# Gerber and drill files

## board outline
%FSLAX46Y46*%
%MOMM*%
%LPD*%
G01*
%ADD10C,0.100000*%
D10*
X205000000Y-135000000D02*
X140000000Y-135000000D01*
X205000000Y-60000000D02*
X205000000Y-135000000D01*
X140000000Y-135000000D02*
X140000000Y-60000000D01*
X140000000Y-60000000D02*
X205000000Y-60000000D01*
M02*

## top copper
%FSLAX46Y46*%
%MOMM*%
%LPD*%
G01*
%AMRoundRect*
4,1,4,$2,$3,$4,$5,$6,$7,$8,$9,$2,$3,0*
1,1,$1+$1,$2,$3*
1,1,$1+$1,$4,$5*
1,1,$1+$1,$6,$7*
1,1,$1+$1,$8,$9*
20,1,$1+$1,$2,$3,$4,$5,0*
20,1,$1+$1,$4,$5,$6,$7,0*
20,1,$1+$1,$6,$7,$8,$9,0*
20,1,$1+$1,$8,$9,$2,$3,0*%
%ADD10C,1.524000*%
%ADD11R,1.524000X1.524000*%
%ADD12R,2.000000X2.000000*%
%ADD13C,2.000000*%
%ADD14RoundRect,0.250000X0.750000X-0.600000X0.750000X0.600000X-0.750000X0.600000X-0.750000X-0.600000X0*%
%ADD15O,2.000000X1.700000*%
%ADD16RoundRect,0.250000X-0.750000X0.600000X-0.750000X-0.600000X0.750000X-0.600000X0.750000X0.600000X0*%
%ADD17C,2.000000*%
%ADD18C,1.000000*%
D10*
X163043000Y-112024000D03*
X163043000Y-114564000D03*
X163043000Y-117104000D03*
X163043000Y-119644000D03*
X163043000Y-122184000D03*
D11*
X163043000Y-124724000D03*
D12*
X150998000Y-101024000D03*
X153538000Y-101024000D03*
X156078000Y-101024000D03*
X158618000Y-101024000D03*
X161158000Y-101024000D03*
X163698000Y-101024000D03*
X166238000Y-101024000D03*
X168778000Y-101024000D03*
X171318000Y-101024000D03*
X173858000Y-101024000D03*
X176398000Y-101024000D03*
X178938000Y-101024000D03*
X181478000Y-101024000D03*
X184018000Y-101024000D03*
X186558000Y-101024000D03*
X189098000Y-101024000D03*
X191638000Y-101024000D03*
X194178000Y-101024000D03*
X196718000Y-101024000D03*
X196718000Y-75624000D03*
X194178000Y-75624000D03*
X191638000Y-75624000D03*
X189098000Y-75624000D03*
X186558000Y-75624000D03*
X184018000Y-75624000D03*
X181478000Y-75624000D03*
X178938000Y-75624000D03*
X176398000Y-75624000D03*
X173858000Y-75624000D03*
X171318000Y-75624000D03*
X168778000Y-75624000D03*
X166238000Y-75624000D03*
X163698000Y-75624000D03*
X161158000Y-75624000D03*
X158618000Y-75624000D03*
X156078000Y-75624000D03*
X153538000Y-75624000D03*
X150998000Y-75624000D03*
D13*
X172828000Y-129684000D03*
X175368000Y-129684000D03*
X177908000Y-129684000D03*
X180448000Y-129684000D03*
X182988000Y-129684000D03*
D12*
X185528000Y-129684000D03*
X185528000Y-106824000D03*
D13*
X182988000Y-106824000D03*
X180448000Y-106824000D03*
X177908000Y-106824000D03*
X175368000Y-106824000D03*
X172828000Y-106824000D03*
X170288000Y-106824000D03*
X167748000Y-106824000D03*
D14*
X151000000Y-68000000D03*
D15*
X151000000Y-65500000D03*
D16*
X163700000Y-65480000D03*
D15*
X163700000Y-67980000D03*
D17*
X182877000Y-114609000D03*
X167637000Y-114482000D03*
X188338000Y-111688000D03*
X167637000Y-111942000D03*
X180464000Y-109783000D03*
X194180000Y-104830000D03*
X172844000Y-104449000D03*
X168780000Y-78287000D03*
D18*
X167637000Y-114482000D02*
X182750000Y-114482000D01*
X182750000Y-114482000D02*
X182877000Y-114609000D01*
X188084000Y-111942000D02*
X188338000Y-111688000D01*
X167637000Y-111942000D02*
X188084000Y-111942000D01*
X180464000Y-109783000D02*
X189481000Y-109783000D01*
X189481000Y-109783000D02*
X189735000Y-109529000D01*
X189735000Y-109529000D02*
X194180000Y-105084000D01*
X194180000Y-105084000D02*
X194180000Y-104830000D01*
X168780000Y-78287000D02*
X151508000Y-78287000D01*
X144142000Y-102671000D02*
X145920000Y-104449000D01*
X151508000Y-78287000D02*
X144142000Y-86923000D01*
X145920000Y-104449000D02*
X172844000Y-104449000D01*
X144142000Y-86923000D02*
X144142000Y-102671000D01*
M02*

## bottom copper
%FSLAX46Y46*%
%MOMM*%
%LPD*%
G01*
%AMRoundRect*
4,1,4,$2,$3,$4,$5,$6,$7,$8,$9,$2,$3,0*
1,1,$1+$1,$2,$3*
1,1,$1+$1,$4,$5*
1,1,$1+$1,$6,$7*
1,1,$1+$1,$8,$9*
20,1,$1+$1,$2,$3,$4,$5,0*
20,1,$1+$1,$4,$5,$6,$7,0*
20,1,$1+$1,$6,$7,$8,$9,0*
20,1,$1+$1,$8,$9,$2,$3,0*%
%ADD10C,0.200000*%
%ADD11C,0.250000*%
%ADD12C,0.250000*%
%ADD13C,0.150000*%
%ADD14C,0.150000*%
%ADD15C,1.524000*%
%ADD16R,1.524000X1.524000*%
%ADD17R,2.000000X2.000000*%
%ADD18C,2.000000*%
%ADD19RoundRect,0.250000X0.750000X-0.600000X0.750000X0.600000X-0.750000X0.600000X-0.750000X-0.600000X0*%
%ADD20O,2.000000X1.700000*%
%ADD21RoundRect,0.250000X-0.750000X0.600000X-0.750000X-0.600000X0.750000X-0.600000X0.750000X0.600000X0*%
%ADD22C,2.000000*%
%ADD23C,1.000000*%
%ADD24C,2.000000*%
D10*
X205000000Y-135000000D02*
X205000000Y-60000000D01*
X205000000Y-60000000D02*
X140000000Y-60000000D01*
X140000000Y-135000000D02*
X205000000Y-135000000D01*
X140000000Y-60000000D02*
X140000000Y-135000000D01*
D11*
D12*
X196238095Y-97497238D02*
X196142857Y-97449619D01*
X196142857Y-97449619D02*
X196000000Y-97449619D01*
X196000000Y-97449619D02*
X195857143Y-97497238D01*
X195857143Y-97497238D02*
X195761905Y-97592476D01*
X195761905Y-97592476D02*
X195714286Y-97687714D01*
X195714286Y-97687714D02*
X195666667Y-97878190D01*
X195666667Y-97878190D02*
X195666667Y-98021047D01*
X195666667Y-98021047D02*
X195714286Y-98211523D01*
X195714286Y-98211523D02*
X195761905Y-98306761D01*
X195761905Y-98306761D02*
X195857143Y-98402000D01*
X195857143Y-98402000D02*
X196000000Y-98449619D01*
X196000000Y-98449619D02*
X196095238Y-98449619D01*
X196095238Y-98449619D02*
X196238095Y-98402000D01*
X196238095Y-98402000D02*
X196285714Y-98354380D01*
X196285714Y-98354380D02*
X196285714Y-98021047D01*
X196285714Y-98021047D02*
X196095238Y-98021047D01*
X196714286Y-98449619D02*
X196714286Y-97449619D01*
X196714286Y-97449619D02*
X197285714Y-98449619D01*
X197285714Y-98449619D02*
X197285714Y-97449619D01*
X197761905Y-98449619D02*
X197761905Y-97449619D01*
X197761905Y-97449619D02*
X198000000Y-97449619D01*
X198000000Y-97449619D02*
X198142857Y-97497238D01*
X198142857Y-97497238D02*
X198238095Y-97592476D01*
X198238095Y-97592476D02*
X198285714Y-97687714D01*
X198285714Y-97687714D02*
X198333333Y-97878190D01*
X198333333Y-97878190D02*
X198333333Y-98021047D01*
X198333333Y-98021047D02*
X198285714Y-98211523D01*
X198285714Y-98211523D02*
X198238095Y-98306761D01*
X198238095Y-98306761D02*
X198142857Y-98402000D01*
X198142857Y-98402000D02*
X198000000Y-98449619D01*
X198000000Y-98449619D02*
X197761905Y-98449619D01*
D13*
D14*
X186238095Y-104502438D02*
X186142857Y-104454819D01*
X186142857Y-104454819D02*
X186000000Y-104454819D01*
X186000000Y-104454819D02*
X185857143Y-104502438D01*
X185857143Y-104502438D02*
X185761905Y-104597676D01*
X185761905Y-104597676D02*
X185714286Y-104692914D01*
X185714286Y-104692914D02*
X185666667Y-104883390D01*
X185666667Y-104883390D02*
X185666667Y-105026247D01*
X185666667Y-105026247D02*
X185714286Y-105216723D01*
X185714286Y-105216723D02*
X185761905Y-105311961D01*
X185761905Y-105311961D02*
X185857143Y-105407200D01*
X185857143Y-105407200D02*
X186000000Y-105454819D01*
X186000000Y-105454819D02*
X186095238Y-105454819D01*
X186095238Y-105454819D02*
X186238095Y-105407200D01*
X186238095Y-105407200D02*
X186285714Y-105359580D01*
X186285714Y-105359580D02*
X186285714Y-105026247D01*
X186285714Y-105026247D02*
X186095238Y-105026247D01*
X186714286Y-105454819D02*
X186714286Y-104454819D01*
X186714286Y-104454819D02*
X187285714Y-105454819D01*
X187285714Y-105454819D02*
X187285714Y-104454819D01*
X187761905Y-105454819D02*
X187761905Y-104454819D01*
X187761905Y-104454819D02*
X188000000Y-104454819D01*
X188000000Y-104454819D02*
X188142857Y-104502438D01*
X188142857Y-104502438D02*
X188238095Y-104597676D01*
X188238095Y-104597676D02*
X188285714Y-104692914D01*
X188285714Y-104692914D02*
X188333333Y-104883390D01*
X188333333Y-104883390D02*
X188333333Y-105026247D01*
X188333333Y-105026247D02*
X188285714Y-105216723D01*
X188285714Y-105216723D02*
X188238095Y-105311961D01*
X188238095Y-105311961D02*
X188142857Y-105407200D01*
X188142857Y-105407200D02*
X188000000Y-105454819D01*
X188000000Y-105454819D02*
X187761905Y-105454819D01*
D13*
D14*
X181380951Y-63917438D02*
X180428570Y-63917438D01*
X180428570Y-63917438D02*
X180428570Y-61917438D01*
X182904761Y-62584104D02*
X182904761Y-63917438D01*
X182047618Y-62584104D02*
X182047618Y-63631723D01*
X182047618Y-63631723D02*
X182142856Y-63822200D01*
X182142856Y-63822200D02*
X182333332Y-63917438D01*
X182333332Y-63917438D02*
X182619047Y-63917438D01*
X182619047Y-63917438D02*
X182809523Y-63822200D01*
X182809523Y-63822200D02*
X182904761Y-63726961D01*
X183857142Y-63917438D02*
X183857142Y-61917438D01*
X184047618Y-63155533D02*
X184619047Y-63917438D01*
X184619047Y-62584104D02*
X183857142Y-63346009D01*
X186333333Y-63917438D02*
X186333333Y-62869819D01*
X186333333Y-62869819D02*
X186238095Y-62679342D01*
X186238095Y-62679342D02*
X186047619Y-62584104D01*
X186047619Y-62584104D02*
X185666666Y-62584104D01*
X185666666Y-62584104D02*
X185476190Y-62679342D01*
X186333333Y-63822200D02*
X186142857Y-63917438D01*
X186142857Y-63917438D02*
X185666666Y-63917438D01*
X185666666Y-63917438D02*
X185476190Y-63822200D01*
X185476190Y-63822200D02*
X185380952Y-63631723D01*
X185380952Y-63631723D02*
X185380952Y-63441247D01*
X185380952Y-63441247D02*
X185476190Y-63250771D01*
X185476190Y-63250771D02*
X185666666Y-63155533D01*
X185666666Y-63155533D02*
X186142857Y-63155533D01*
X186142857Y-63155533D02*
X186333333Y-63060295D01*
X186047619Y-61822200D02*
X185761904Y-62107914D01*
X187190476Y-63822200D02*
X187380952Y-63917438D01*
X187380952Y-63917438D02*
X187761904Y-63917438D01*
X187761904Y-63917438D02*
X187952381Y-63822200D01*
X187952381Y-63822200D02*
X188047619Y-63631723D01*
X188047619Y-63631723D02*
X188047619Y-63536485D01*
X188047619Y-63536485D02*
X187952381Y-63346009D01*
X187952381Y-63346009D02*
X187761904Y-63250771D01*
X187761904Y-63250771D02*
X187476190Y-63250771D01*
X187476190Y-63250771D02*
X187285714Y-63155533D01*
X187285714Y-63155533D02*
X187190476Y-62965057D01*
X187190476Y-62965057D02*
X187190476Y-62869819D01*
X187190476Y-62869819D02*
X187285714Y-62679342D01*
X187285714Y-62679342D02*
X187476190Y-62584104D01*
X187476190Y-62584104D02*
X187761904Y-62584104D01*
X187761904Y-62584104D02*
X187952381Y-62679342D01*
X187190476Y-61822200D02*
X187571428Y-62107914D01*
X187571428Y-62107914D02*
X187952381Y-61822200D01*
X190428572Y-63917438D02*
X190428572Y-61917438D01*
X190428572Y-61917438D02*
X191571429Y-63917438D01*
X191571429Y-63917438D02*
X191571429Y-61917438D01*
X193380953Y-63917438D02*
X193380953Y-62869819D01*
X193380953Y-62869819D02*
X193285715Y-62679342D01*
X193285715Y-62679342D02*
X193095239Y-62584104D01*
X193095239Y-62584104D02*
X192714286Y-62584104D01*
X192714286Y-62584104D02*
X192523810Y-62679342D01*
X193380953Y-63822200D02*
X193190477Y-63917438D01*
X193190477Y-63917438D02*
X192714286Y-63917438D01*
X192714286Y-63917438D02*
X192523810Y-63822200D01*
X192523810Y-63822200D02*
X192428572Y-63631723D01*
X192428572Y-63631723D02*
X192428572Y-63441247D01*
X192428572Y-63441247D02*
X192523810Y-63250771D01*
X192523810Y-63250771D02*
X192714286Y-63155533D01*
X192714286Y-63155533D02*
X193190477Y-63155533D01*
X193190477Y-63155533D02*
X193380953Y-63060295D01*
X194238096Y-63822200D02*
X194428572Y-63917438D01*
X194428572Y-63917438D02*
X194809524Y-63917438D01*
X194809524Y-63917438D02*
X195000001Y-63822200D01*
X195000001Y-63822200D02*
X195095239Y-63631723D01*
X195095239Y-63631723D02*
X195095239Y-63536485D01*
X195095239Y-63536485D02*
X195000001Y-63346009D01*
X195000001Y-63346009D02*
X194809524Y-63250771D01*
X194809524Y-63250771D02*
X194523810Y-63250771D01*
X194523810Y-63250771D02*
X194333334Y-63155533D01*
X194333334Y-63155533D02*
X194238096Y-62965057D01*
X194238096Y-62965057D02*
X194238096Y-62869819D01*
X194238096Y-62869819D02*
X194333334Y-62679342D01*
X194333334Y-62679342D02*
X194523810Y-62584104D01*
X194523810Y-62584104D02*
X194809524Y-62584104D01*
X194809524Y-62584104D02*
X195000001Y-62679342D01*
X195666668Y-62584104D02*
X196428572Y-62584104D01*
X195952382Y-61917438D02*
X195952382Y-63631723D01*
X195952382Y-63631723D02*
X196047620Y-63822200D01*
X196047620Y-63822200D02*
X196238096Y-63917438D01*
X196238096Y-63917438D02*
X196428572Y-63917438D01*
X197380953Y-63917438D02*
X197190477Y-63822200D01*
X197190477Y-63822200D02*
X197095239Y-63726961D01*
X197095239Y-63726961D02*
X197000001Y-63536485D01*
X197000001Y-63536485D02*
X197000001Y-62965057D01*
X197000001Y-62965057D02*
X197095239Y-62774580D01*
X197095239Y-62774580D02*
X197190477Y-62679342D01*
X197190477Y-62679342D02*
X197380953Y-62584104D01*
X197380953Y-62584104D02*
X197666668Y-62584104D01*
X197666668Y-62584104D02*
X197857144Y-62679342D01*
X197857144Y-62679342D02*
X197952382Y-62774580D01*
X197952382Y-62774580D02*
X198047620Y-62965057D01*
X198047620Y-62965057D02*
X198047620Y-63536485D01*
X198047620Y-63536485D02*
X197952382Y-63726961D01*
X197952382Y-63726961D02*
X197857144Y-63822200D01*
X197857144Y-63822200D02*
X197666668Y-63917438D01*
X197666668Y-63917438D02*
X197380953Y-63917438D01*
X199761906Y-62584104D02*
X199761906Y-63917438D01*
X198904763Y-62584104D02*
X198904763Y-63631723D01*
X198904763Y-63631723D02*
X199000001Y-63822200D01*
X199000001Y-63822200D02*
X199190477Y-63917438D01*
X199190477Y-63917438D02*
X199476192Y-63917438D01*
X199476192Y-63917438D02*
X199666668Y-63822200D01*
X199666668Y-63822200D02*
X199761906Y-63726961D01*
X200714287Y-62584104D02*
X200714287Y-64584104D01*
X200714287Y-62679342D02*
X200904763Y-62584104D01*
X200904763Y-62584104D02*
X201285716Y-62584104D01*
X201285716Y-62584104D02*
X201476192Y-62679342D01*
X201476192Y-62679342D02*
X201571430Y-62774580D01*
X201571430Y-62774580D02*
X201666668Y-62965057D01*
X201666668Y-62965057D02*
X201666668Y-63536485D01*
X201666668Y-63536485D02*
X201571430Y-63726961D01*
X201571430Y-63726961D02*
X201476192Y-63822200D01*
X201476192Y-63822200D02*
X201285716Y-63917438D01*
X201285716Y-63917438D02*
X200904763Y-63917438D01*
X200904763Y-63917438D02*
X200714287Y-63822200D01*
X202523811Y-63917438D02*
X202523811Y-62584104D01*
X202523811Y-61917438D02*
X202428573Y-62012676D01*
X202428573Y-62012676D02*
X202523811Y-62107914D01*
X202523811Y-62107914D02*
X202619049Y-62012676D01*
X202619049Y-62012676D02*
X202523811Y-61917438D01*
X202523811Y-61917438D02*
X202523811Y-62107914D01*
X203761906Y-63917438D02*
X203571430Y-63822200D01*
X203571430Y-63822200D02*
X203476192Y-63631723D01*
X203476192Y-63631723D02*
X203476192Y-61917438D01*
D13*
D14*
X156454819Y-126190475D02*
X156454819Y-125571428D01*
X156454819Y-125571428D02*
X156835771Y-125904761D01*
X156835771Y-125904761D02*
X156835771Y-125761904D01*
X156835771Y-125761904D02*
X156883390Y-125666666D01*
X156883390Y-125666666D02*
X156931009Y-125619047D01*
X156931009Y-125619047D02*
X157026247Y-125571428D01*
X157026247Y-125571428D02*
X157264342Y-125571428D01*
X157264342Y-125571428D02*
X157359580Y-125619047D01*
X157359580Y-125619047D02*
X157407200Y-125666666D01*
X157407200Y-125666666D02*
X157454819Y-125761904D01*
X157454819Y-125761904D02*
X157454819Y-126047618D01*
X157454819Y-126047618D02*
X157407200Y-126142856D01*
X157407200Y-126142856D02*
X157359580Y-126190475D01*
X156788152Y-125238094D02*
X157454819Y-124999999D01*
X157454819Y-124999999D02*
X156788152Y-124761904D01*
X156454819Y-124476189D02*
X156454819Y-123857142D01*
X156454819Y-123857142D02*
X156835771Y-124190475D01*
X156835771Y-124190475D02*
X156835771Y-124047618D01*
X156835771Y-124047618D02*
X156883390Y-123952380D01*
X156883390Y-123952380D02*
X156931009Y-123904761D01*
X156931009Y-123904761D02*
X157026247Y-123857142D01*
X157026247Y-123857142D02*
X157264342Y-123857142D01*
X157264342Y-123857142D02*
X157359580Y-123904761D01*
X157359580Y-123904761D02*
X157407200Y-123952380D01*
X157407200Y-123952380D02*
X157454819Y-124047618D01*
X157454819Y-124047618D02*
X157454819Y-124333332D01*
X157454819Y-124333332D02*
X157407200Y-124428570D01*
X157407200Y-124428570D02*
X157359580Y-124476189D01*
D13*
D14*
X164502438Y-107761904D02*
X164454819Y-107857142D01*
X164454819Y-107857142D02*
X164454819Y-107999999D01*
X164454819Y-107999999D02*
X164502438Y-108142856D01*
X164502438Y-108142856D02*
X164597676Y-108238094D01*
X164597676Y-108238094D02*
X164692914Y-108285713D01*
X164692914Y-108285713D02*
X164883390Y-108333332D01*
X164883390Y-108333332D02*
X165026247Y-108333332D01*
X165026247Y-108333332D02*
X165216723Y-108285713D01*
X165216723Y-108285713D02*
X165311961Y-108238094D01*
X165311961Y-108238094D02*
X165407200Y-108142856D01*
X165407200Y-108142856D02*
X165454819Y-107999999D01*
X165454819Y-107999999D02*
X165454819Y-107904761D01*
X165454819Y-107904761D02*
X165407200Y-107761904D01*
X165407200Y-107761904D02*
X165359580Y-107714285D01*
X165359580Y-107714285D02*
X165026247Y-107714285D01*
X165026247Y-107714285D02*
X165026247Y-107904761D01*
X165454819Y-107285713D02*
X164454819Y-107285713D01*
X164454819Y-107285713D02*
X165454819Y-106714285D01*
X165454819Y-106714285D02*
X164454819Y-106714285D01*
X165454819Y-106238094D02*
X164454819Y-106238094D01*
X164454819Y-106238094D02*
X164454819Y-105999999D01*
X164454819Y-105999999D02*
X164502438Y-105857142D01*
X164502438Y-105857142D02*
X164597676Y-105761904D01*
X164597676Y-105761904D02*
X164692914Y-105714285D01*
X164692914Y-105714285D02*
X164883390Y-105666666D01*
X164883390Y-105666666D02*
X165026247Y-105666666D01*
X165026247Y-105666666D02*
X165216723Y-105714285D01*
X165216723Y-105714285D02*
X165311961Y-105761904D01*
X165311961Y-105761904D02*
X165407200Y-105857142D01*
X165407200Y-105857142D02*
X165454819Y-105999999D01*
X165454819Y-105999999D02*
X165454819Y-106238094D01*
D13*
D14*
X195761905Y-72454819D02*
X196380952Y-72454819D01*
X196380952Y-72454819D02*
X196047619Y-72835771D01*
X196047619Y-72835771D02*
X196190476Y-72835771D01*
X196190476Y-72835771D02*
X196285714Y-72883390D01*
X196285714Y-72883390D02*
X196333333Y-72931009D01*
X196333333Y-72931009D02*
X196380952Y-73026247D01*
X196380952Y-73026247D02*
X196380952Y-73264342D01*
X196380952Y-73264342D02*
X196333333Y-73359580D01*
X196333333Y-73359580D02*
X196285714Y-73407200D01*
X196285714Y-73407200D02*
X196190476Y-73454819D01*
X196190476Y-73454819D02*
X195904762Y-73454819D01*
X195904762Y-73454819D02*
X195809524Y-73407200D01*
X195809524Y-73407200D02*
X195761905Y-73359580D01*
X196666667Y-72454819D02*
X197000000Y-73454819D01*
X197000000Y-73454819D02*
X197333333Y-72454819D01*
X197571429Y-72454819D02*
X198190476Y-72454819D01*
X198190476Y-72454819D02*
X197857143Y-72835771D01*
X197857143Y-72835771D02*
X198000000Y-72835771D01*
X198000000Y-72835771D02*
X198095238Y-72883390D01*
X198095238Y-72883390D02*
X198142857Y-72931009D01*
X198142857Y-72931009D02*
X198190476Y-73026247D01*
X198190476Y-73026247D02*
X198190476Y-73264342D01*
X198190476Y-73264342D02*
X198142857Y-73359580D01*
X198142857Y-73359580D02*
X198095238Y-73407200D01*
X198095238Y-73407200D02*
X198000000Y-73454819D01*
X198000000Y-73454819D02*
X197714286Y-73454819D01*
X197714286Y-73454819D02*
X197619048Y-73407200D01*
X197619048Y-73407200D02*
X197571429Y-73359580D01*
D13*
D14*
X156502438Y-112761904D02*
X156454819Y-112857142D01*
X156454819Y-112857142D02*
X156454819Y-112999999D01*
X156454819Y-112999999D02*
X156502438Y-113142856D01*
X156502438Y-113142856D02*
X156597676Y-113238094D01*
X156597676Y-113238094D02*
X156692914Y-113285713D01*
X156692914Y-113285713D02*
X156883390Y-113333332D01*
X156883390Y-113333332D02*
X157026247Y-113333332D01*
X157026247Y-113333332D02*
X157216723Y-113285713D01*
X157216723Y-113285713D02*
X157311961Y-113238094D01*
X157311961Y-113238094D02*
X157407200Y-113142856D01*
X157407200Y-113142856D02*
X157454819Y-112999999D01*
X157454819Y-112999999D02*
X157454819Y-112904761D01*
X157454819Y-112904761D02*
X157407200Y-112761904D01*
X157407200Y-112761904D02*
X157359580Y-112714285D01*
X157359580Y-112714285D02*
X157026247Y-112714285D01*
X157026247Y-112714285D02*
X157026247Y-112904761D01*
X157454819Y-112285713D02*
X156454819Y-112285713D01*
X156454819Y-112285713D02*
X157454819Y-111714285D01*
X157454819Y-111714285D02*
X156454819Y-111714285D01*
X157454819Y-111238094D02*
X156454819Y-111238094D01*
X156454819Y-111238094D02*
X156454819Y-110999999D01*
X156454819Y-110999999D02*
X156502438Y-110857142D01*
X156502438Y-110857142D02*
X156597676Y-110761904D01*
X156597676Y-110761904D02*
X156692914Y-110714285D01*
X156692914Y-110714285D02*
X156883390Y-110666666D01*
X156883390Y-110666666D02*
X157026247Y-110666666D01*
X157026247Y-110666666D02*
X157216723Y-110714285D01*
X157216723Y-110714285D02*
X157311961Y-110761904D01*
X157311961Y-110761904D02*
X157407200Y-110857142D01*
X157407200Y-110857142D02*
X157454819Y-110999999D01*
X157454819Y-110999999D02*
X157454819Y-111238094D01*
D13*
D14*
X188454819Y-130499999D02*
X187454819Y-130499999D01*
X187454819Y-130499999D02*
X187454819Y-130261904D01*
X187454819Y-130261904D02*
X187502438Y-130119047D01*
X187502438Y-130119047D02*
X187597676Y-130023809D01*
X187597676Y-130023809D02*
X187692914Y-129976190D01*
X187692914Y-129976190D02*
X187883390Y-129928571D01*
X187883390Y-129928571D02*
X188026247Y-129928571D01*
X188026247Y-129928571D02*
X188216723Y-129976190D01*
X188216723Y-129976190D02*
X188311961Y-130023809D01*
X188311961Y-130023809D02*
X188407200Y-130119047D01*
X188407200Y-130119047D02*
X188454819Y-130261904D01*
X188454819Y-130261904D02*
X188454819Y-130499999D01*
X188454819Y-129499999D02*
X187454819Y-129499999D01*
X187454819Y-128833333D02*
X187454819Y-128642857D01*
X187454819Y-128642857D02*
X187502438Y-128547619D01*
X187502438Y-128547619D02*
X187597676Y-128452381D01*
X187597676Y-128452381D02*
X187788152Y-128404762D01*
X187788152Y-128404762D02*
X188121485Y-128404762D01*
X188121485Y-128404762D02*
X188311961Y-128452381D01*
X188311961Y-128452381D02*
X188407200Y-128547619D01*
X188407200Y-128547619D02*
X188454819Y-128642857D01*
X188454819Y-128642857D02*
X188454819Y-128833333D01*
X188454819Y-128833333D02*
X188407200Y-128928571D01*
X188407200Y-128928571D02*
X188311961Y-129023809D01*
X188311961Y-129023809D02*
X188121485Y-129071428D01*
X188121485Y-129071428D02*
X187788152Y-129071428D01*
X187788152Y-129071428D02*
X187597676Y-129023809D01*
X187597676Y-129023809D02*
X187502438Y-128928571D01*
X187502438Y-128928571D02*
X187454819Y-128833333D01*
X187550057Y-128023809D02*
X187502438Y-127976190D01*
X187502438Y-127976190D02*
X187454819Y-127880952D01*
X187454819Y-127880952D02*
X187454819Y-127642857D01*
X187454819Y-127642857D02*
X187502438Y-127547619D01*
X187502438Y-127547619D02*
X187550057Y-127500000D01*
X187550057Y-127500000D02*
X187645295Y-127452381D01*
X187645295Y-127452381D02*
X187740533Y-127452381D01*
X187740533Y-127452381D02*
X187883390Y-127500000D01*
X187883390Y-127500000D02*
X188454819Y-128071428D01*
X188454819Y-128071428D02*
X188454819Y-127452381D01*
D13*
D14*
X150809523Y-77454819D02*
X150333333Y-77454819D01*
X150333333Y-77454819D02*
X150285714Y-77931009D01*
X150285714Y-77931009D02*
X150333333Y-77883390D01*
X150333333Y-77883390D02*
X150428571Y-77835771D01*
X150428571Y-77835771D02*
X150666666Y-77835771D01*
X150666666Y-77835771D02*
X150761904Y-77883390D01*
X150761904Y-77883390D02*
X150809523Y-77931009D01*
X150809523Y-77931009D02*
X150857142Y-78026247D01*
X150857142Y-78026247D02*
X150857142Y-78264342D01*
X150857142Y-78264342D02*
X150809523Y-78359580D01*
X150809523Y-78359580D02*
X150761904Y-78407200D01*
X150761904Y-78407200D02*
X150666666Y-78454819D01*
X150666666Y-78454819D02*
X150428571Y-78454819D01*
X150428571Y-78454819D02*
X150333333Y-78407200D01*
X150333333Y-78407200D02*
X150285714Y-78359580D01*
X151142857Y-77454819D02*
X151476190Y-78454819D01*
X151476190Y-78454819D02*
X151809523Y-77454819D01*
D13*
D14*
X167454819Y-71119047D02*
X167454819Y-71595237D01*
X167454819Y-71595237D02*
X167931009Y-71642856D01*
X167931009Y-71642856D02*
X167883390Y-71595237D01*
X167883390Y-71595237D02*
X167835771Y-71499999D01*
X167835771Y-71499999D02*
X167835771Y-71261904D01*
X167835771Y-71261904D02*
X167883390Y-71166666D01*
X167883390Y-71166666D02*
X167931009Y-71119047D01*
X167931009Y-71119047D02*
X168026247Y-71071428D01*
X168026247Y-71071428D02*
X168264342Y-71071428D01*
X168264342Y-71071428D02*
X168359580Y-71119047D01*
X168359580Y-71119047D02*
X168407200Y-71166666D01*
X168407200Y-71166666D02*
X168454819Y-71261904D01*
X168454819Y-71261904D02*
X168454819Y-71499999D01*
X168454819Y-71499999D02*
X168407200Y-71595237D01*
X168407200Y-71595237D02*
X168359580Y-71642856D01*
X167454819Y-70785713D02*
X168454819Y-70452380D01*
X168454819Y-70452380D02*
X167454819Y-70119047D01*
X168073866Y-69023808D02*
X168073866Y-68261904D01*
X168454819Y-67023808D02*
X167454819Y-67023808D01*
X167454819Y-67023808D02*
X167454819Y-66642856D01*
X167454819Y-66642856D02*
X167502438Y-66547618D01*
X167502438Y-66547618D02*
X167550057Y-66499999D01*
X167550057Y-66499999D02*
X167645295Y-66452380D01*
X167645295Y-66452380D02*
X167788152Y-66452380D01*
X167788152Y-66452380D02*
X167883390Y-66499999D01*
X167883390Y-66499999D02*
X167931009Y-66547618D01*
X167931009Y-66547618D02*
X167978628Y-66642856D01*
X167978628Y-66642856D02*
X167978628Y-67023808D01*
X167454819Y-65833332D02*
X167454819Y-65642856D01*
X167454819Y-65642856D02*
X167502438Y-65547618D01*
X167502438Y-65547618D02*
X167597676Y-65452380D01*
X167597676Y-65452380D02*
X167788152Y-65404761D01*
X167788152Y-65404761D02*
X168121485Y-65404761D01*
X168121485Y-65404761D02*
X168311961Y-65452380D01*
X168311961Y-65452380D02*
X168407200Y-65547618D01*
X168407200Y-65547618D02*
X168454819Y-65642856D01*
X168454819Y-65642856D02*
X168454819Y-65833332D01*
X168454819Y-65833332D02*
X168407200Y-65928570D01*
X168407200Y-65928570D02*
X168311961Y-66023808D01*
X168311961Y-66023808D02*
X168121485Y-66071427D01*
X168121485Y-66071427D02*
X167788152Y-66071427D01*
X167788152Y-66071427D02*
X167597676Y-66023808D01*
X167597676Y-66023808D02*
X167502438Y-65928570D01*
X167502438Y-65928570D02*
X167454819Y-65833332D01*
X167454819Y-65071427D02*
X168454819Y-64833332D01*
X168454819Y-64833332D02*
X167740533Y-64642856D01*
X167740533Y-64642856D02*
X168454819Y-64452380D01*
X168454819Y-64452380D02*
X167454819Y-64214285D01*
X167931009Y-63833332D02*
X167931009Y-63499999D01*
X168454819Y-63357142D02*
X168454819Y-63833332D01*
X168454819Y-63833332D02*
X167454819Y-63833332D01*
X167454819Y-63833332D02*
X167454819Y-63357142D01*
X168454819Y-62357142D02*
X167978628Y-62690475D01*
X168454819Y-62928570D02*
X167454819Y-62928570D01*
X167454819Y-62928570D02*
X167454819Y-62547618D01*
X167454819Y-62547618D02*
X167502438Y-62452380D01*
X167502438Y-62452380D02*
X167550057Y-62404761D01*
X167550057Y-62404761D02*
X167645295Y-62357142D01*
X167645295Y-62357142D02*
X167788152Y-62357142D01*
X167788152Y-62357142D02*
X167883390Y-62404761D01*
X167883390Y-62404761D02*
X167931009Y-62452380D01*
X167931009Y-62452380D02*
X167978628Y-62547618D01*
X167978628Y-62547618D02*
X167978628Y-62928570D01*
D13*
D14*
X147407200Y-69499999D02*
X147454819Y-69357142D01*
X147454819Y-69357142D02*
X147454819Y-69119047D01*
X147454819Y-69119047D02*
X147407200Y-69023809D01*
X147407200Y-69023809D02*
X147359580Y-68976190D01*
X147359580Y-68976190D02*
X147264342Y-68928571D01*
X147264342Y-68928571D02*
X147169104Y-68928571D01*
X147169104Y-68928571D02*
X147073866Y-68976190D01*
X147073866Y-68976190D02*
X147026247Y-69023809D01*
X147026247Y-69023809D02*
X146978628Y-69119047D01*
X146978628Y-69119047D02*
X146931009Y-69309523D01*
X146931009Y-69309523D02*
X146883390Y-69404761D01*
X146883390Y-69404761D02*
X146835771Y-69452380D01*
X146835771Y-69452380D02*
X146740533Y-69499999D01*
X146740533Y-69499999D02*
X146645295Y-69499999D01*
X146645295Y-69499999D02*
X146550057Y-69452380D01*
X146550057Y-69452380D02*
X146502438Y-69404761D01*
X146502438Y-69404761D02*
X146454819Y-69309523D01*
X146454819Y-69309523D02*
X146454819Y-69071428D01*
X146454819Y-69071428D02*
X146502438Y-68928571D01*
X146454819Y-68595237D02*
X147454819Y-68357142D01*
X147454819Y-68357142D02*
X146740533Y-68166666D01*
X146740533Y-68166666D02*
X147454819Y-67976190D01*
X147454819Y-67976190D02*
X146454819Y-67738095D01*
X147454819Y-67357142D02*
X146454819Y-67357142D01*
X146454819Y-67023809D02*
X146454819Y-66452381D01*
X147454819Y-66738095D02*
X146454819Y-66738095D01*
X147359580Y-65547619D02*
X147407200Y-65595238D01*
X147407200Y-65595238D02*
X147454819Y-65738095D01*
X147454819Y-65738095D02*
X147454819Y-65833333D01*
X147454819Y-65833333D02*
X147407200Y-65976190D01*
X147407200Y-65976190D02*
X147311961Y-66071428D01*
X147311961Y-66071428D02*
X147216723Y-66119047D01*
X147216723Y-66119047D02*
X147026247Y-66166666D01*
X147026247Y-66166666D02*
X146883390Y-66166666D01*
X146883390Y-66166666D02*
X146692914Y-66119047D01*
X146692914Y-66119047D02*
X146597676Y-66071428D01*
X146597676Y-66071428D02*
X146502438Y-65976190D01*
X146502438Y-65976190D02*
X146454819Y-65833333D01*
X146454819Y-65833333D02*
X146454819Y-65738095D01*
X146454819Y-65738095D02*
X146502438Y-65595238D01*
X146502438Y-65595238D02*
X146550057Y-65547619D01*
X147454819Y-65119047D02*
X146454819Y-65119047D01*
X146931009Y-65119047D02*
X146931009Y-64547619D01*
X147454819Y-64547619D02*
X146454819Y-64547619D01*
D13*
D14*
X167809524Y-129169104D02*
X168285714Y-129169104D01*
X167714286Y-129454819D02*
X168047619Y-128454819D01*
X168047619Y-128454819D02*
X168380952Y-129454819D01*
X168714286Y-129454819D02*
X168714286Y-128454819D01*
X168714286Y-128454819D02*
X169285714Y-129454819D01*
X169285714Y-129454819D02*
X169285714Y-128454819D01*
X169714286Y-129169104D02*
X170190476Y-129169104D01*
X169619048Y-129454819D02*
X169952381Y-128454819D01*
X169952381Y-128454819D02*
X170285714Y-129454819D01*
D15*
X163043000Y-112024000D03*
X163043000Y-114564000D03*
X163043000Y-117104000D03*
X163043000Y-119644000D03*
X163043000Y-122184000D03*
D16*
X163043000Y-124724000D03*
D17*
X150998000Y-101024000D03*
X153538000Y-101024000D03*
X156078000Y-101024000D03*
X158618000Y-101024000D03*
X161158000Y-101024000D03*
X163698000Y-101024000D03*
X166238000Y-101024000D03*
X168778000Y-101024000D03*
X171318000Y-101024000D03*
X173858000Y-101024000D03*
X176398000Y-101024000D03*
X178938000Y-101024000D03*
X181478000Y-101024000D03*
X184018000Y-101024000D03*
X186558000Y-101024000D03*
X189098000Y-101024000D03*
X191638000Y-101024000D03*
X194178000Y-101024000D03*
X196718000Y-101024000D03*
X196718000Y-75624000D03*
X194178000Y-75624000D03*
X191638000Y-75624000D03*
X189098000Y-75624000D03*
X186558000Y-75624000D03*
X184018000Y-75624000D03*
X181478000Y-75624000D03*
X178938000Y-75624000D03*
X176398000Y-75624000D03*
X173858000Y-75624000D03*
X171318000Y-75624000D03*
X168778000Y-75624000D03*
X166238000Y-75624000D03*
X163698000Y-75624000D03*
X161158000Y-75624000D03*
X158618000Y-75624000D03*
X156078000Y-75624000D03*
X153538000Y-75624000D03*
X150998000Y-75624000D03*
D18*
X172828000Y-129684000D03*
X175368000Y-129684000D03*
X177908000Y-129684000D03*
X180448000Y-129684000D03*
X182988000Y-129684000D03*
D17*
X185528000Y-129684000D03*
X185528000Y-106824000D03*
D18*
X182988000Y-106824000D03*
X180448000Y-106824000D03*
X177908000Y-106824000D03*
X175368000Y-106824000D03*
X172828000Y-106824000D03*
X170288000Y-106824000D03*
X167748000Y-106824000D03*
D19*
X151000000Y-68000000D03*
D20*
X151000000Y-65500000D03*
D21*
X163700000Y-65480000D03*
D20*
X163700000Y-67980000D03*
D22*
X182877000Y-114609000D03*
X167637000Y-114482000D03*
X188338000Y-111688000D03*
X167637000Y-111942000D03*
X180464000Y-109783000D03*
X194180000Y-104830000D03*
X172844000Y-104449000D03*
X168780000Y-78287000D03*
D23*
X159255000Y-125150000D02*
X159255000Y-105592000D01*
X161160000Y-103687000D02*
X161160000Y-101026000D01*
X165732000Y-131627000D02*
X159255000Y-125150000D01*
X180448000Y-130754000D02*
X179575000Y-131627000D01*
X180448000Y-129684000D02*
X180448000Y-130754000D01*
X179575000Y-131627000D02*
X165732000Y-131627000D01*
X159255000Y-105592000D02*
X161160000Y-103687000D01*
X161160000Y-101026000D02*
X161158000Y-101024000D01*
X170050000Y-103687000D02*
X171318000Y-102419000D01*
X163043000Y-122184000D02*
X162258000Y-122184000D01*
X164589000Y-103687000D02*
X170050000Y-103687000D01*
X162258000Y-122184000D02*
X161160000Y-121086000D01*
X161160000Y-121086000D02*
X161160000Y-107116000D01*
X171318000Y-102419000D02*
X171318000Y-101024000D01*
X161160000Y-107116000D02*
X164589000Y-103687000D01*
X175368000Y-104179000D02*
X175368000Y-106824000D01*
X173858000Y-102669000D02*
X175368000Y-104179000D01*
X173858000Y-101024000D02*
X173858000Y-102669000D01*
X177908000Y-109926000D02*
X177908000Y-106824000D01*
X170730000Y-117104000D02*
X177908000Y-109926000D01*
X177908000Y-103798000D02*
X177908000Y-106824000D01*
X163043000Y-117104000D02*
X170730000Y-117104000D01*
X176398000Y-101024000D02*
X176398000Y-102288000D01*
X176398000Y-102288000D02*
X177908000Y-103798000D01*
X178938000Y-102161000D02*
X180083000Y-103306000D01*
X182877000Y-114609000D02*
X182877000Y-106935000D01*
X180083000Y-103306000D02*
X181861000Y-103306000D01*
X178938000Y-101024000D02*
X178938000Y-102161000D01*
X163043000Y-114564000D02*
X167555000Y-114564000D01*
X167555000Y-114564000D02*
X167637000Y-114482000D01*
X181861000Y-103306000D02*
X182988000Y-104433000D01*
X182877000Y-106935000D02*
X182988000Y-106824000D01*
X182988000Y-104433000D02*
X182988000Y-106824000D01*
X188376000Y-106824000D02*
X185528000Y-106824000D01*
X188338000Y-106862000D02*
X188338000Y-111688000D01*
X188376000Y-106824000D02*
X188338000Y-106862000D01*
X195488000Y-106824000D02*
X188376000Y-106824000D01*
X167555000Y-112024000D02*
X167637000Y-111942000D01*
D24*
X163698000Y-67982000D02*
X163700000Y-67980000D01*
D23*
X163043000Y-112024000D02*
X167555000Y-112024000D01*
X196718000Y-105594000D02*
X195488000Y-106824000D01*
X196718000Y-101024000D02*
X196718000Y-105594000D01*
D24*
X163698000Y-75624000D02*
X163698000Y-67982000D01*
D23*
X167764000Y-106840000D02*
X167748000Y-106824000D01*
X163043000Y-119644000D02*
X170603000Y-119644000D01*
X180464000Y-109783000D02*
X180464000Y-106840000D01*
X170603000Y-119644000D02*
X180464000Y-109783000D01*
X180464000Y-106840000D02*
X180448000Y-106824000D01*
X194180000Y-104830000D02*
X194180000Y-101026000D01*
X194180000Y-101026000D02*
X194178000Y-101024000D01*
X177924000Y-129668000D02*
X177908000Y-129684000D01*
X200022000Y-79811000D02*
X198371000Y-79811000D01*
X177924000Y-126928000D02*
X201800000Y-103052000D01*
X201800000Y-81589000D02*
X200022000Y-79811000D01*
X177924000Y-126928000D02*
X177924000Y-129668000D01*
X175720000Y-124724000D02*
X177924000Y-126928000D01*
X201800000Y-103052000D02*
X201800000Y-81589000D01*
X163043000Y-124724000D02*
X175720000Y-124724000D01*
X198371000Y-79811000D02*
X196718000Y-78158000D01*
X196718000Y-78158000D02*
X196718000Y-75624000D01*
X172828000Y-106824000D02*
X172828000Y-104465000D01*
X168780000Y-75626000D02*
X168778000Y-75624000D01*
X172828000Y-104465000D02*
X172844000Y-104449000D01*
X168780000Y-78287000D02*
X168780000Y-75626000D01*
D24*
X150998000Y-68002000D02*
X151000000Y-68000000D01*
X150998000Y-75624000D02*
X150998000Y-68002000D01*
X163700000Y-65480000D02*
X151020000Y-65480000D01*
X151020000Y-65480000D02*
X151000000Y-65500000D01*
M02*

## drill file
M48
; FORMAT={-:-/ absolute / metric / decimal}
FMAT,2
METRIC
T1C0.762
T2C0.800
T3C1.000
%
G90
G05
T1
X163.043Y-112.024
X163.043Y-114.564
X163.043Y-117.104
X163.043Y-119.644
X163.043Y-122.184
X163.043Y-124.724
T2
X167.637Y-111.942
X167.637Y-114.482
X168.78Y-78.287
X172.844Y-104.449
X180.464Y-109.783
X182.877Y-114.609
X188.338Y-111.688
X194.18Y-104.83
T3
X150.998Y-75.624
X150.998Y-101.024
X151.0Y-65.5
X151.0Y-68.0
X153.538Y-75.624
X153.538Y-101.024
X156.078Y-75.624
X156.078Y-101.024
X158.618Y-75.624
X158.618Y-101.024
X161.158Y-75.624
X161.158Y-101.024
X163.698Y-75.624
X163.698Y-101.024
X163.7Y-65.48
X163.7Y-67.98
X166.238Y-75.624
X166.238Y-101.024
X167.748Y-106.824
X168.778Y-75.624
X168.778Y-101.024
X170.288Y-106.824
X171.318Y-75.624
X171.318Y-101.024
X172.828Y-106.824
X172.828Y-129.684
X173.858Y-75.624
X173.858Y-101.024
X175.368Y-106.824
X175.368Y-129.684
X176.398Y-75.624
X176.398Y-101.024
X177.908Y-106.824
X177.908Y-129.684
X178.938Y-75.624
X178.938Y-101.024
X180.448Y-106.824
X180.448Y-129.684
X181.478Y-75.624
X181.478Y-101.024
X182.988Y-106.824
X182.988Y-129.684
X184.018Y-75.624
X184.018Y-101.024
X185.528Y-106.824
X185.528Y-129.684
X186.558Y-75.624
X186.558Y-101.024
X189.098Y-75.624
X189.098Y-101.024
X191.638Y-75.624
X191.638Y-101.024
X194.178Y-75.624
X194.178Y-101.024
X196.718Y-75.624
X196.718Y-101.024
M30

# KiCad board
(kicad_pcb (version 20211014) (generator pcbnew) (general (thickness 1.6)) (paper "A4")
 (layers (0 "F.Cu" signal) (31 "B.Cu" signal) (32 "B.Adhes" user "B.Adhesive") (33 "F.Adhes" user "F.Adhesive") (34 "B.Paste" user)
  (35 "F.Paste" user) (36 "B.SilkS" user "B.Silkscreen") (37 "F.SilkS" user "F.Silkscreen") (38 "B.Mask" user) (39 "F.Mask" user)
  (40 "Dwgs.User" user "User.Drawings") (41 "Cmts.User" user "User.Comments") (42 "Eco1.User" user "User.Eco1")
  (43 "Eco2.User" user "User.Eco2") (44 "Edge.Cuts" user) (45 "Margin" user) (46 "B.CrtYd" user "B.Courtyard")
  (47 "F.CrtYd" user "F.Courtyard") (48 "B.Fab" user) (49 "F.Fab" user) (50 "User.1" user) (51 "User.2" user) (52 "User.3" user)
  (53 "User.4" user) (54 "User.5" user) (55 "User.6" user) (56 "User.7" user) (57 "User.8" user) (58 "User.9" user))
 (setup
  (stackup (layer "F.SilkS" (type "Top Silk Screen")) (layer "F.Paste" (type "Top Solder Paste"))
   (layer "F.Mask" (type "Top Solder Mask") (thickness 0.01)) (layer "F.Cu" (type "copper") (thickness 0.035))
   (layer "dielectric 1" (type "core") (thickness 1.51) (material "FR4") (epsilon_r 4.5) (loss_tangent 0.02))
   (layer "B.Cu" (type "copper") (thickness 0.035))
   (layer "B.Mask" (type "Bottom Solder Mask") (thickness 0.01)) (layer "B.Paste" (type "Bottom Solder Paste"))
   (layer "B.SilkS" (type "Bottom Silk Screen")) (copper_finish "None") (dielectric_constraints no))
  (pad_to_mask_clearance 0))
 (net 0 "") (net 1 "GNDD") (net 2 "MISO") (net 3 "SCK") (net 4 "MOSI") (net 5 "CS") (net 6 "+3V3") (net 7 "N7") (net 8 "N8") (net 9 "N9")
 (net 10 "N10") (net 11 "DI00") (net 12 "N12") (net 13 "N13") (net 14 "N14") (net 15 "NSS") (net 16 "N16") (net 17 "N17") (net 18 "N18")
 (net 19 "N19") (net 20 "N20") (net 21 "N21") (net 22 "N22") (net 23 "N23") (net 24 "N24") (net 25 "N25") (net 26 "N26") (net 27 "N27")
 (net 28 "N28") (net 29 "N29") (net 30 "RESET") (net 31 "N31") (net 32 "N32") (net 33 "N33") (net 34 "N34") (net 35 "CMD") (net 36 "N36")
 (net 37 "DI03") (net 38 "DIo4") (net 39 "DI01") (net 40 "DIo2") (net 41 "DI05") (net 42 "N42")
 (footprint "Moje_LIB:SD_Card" (layer "F.Cu") (at 163.743 110.374 -90)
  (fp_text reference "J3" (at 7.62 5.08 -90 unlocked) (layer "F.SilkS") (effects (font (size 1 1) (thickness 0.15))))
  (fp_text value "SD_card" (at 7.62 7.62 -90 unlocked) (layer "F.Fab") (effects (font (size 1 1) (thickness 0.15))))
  (pad "1" thru_hole circle (at 1.65 0.7 270) (size 1.524 1.524) (drill 0.762) (layers *.Cu *.Mask) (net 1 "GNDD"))
  (pad "2" thru_hole circle (at 4.19 0.7 270) (size 1.524 1.524) (drill 0.762) (layers *.Cu *.Mask) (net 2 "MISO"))
  (pad "3" thru_hole circle (at 6.73 0.7 270) (size 1.524 1.524) (drill 0.762) (layers *.Cu *.Mask) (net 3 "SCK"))
  (pad "4" thru_hole circle (at 9.27 0.7 270) (size 1.524 1.524) (drill 0.762) (layers *.Cu *.Mask) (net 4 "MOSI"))
  (pad "5" thru_hole circle (at 11.81 0.7 270) (size 1.524 1.524) (drill 0.762) (layers *.Cu *.Mask) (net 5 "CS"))
  (pad "6" thru_hole rect (at 14.35 0.7 270) (size 1.524 1.524) (drill 0.762) (layers *.Cu *.Mask) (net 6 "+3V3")))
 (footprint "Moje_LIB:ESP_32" (layer "F.Cu") (at 145.998 74.624)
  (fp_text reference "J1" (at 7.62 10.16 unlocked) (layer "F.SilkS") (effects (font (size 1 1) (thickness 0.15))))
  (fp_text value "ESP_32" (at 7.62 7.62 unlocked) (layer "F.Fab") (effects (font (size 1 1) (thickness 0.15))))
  (pad "1" thru_hole rect (at 5 26.4) (size 2 2) (drill 1) (layers *.Cu *.Mask) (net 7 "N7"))
  (pad "2" thru_hole rect (at 7.54 26.4) (size 2 2) (drill 1) (layers *.Cu *.Mask) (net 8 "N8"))
  (pad "3" thru_hole rect (at 10.08 26.4) (size 2 2) (drill 1) (layers *.Cu *.Mask) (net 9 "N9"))
  (pad "4" thru_hole rect (at 12.62 26.4) (size 2 2) (drill 1) (layers *.Cu *.Mask) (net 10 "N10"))
  (pad "5" thru_hole rect (at 15.16 26.4) (size 2 2) (drill 1) (layers *.Cu *.Mask) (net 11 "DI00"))
  (pad "6" thru_hole rect (at 17.7 26.4) (size 2 2) (drill 1) (layers *.Cu *.Mask) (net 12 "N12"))
  (pad "7" thru_hole rect (at 20.24 26.4) (size 2 2) (drill 1) (layers *.Cu *.Mask) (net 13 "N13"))
  (pad "8" thru_hole rect (at 22.78 26.4) (size 2 2) (drill 1) (layers *.Cu *.Mask) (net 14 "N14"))
  (pad "9" thru_hole rect (at 25.32 26.4) (size 2 2) (drill 1) (layers *.Cu *.Mask) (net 5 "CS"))
  (pad "10" thru_hole rect (at 27.86 26.4) (size 2 2) (drill 1) (layers *.Cu *.Mask) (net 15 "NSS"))
  (pad "11" thru_hole rect (at 30.4 26.4) (size 2 2) (drill 1) (layers *.Cu *.Mask) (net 3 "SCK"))
  (pad "12" thru_hole rect (at 32.94 26.4) (size 2 2) (drill 1) (layers *.Cu *.Mask) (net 2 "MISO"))
  (pad "13" thru_hole rect (at 35.48 26.4) (size 2 2) (drill 1) (layers *.Cu *.Mask) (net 1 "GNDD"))
  (pad "14" thru_hole rect (at 38.02 26.4) (size 2 2) (drill 1) (layers *.Cu *.Mask) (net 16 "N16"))
  (pad "15" thru_hole rect (at 40.56 26.4) (size 2 2) (drill 1) (layers *.Cu *.Mask) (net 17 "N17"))
  (pad "16" thru_hole rect (at 43.1 26.4) (size 2 2) (drill 1) (layers *.Cu *.Mask) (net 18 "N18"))
  (pad "17" thru_hole rect (at 45.64 26.4) (size 2 2) (drill 1) (layers *.Cu *.Mask) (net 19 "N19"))
  (pad "18" thru_hole rect (at 48.18 26.4) (size 2 2) (drill 1) (layers *.Cu *.Mask) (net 4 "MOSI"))
  (pad "19" thru_hole rect (at 50.72 26.4) (size 2 2) (drill 1) (layers *.Cu *.Mask) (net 1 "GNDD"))
  (pad "20" thru_hole rect (at 50.72 1) (size 2 2) (drill 1) (layers *.Cu *.Mask) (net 6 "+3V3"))
  (pad "21" thru_hole rect (at 48.18 1) (size 2 2) (drill 1) (layers *.Cu *.Mask) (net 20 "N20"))
  (pad "22" thru_hole rect (at 45.64 1) (size 2 2) (drill 1) (layers *.Cu *.Mask) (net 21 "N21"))
  (pad "23" thru_hole rect (at 43.1 1) (size 2 2) (drill 1) (layers *.Cu *.Mask) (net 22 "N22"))
  (pad "24" thru_hole rect (at 40.56 1) (size 2 2) (drill 1) (layers *.Cu *.Mask) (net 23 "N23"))
  (pad "25" thru_hole rect (at 38.02 1) (size 2 2) (drill 1) (layers *.Cu *.Mask) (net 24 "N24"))
  (pad "26" thru_hole rect (at 35.48 1) (size 2 2) (drill 1) (layers *.Cu *.Mask) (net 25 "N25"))
  (pad "27" thru_hole rect (at 32.94 1) (size 2 2) (drill 1) (layers *.Cu *.Mask) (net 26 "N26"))
  (pad "28" thru_hole rect (at 30.4 1) (size 2 2) (drill 1) (layers *.Cu *.Mask) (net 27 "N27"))
  (pad "29" thru_hole rect (at 27.86 1) (size 2 2) (drill 1) (layers *.Cu *.Mask) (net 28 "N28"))
  (pad "30" thru_hole rect (at 25.32 1) (size 2 2) (drill 1) (layers *.Cu *.Mask) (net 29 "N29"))
  (pad "31" thru_hole rect (at 22.78 1) (size 2 2) (drill 1) (layers *.Cu *.Mask) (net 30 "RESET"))
  (pad "32" thru_hole rect (at 20.24 1) (size 2 2) (drill 1) (layers *.Cu *.Mask) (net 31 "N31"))
  (pad "33" thru_hole rect (at 17.7 1) (size 2 2) (drill 1) (layers *.Cu *.Mask) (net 1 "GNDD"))
  (pad "34" thru_hole rect (at 15.16 1) (size 2 2) (drill 1) (layers *.Cu *.Mask) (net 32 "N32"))
  (pad "35" thru_hole rect (at 12.62 1) (size 2 2) (drill 1) (layers *.Cu *.Mask) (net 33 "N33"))
  (pad "36" thru_hole rect (at 10.08 1) (size 2 2) (drill 1) (layers *.Cu *.Mask) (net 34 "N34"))
  (pad "37" thru_hole rect (at 7.54 1) (size 2 2) (drill 1) (layers *.Cu *.Mask) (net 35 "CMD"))
  (pad "38" thru_hole rect (at 5 1) (size 2 2) (drill 1) (layers *.Cu *.Mask) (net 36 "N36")))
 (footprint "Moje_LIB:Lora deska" (layer "F.Cu") (at 165.498 131.684 90)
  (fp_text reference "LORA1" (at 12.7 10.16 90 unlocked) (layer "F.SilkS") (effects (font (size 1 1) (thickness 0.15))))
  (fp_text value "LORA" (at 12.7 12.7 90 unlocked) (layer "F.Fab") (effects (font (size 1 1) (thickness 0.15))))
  (pad "3" thru_hole circle (at 2 7.33 90) (size 2 2) (drill 1) (layers *.Cu *.Mask) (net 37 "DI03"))
  (pad "4" thru_hole circle (at 2 9.87 90) (size 2 2) (drill 1) (layers *.Cu *.Mask) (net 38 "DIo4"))
  (pad "5" thru_hole circle (at 2 12.41 90) (size 2 2) (drill 1) (layers *.Cu *.Mask) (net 6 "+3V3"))
  (pad "6" thru_hole circle (at 2 14.95 90) (size 2 2) (drill 1) (layers *.Cu *.Mask) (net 11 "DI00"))
  (pad "7" thru_hole circle (at 2 17.49 90) (size 2 2) (drill 1) (layers *.Cu *.Mask) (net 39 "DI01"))
  (pad "8" thru_hole rect (at 2 20.03 90) (size 2 2) (drill 1) (layers *.Cu *.Mask) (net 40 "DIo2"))
  (pad "9" thru_hole rect (at 24.86 20.03 90) (size 2 2) (drill 1) (layers *.Cu *.Mask) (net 1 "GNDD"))
  (pad "10" thru_hole circle (at 24.86 17.49 90) (size 2 2) (drill 1) (layers *.Cu *.Mask) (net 2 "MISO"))
  (pad "11" thru_hole circle (at 24.86 14.95 90) (size 2 2) (drill 1) (layers *.Cu *.Mask) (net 4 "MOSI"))
  (pad "12" thru_hole circle (at 24.86 12.41 90) (size 2 2) (drill 1) (layers *.Cu *.Mask) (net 3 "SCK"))
  (pad "13" thru_hole circle (at 24.86 9.87 90) (size 2 2) (drill 1) (layers *.Cu *.Mask) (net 15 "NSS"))
  (pad "14" thru_hole circle (at 24.86 7.33 90) (size 2 2) (drill 1) (layers *.Cu *.Mask) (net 30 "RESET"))
  (pad "15" thru_hole circle (at 24.86 4.79 90) (size 2 2) (drill 1) (layers *.Cu *.Mask) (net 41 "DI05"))
  (pad "16" thru_hole circle (at 24.86 2.25 90) (size 2 2) (drill 1) (layers *.Cu *.Mask) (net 1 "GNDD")))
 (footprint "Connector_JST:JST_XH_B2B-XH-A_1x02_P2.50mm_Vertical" (layer "F.Cu") (at 151 68 90)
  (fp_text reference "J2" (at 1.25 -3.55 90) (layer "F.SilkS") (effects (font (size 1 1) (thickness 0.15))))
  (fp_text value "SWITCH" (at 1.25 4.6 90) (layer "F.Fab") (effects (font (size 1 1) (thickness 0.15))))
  (pad "1" thru_hole roundrect (at 0 0 90) (size 1.7 2) (drill 1) (layers *.Cu *.Mask) (roundrect_rratio 0.147059) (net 36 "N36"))
  (pad "2" thru_hole oval (at 2.5 0 90) (size 1.7 2) (drill 1) (layers *.Cu *.Mask) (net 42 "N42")))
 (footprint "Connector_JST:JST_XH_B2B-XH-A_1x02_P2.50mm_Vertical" (layer "F.Cu") (at 163.7 65.48 -90)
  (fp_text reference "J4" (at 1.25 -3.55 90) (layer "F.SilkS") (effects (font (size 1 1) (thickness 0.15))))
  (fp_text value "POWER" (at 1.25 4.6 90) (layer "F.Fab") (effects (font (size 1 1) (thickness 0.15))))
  (pad "1" thru_hole roundrect (at 0 0 270) (size 1.7 2) (drill 1) (layers *.Cu *.Mask) (roundrect_rratio 0.147059) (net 42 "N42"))
  (pad "2" thru_hole oval (at 2.5 0 270) (size 1.7 2) (drill 1) (layers *.Cu *.Mask) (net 1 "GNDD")))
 (gr_line (start 205 135) (end 205 60) (layer "B.Cu") (width 0.2))
 (gr_line (start 205 60) (end 140 60) (layer "B.Cu") (width 0.2))
 (gr_line (start 140 135) (end 205 135) (layer "B.Cu") (width 0.2))
 (gr_line (start 140 60) (end 140 135) (layer "B.Cu") (width 0.2))
 (gr_line (start 205 135) (end 140 135) (layer "Edge.Cuts") (width 0.1))
 (gr_line (start 205 60) (end 205 135) (layer "Edge.Cuts") (width 0.1))
 (gr_line (start 140 135) (end 140 60) (layer "Edge.Cuts") (width 0.1))
 (gr_line (start 140 60) (end 205 60) (layer "Edge.Cuts") (width 0.1))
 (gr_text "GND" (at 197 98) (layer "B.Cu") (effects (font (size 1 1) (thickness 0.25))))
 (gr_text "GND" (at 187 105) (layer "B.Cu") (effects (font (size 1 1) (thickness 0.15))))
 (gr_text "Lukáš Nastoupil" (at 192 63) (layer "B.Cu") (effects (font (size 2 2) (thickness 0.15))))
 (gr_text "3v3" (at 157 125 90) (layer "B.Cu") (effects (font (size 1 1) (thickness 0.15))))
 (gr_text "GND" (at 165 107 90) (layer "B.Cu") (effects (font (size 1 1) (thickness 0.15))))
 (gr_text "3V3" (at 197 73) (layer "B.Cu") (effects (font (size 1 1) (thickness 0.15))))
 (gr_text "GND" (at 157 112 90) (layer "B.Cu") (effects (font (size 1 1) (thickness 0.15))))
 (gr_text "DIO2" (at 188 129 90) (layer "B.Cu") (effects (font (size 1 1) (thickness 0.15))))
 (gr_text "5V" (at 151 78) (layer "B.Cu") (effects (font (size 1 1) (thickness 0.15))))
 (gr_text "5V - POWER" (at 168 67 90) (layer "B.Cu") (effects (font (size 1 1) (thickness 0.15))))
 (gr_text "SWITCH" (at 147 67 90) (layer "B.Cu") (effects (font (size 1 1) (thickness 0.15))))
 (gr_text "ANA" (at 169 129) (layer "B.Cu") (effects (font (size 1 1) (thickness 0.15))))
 (segment (start 159.255 125.15) (end 159.255 105.592) (width 1) (layer "B.Cu") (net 11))
 (segment (start 161.16 103.687) (end 161.16 101.026) (width 1) (layer "B.Cu") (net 11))
 (segment (start 165.732 131.627) (end 159.255 125.15) (width 1) (layer "B.Cu") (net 11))
 (segment (start 180.448 130.754) (end 179.575 131.627) (width 1) (layer "B.Cu") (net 11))
 (segment (start 180.448 129.684) (end 180.448 130.754) (width 1) (layer "B.Cu") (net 11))
 (segment (start 179.575 131.627) (end 165.732 131.627) (width 1) (layer "B.Cu") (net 11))
 (segment (start 159.255 105.592) (end 161.16 103.687) (width 1) (layer "B.Cu") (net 11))
 (segment (start 161.16 101.026) (end 161.158 101.024) (width 1) (layer "B.Cu") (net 11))
 (segment (start 170.05 103.687) (end 171.318 102.419) (width 1) (layer "B.Cu") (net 5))
 (segment (start 163.043 122.184) (end 162.258 122.184) (width 1) (layer "B.Cu") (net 5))
 (segment (start 164.589 103.687) (end 170.05 103.687) (width 1) (layer "B.Cu") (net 5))
 (segment (start 162.258 122.184) (end 161.16 121.086) (width 1) (layer "B.Cu") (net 5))
 (segment (start 161.16 121.086) (end 161.16 107.116) (width 1) (layer "B.Cu") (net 5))
 (segment (start 171.318 102.419) (end 171.318 101.024) (width 1) (layer "B.Cu") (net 5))
 (segment (start 161.16 107.116) (end 164.589 103.687) (width 1) (layer "B.Cu") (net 5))
 (segment (start 175.368 104.179) (end 175.368 106.824) (width 1) (layer "B.Cu") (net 15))
 (segment (start 173.858 102.669) (end 175.368 104.179) (width 1) (layer "B.Cu") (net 15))
 (segment (start 173.858 101.024) (end 173.858 102.669) (width 1) (layer "B.Cu") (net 15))
 (segment (start 177.908 109.926) (end 177.908 106.824) (width 1) (layer "B.Cu") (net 3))
 (segment (start 170.73 117.104) (end 177.908 109.926) (width 1) (layer "B.Cu") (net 3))
 (segment (start 177.908 103.798) (end 177.908 106.824) (width 1) (layer "B.Cu") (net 3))
 (segment (start 163.043 117.104) (end 170.73 117.104) (width 1) (layer "B.Cu") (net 3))
 (segment (start 176.398 101.024) (end 176.398 102.288) (width 1) (layer "B.Cu") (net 3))
 (segment (start 176.398 102.288) (end 177.908 103.798) (width 1) (layer "B.Cu") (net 3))
 (segment (start 167.637 114.482) (end 182.75 114.482) (width 1) (layer "F.Cu") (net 2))
 (segment (start 182.75 114.482) (end 182.877 114.609) (width 1) (layer "F.Cu") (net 2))
 (via (at 182.877 114.609) (size 2) (drill 0.8) (layers "F.Cu" "B.Cu") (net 2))
 (via (at 167.637 114.482) (size 2) (drill 0.8) (layers "F.Cu" "B.Cu") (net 2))
 (segment (start 178.938 102.161) (end 180.083 103.306) (width 1) (layer "B.Cu") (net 2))
 (segment (start 182.877 114.609) (end 182.877 106.935) (width 1) (layer "B.Cu") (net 2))
 (segment (start 180.083 103.306) (end 181.861 103.306) (width 1) (layer "B.Cu") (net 2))
 (segment (start 178.938 101.024) (end 178.938 102.161) (width 1) (layer "B.Cu") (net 2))
 (segment (start 163.043 114.564) (end 167.555 114.564) (width 1) (layer "B.Cu") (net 2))
 (segment (start 167.555 114.564) (end 167.637 114.482) (width 1) (layer "B.Cu") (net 2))
 (segment (start 181.861 103.306) (end 182.988 104.433) (width 1) (layer "B.Cu") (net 2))
 (segment (start 182.877 106.935) (end 182.988 106.824) (width 1) (layer "B.Cu") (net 2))
 (segment (start 182.988 104.433) (end 182.988 106.824) (width 1) (layer "B.Cu") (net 2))
 (segment (start 188.084 111.942) (end 188.338 111.688) (width 1) (layer "F.Cu") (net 1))
 (segment (start 167.637 111.942) (end 188.084 111.942) (width 1) (layer "F.Cu") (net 1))
 (via (at 188.338 111.688) (size 2) (drill 0.8) (layers "F.Cu" "B.Cu") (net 1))
 (via (at 167.637 111.942) (size 2) (drill 0.8) (layers "F.Cu" "B.Cu") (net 1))
 (segment (start 188.376 106.824) (end 185.528 106.824) (width 1) (layer "B.Cu") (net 1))
 (segment (start 188.338 106.862) (end 188.338 111.688) (width 1) (layer "B.Cu") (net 1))
 (segment (start 188.376 106.824) (end 188.338 106.862) (width 1) (layer "B.Cu") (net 1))
 (segment (start 195.488 106.824) (end 188.376 106.824) (width 1) (layer "B.Cu") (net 1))
 (segment (start 167.555 112.024) (end 167.637 111.942) (width 1) (layer "B.Cu") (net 1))
 (segment (start 163.698 67.982) (end 163.7 67.98) (width 2) (layer "B.Cu") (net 1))
 (segment (start 163.043 112.024) (end 167.555 112.024) (width 1) (layer "B.Cu") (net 1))
 (segment (start 196.718 105.594) (end 195.488 106.824) (width 1) (layer "B.Cu") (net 1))
 (segment (start 196.718 101.024) (end 196.718 105.594) (width 1) (layer "B.Cu") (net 1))
 (segment (start 163.698 75.624) (end 163.698 67.982) (width 2) (layer "B.Cu") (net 1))
 (segment (start 167.764 106.84) (end 167.748 106.824) (width 1) (layer "B.Cu") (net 1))
 (segment (start 180.464 109.783) (end 189.481 109.783) (width 1) (layer "F.Cu") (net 4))
 (segment (start 189.481 109.783) (end 189.735 109.529) (width 1) (layer "F.Cu") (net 4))
 (segment (start 189.735 109.529) (end 194.18 105.084) (width 1) (layer "F.Cu") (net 4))
 (segment (start 194.18 105.084) (end 194.18 104.83) (width 1) (layer "F.Cu") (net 4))
 (via (at 180.464 109.783) (size 2) (drill 0.8) (layers "F.Cu" "B.Cu") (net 4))
 (via (at 194.18 104.83) (size 2) (drill 0.8) (layers "F.Cu" "B.Cu") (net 4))
 (segment (start 163.043 119.644) (end 170.603 119.644) (width 1) (layer "B.Cu") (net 4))
 (segment (start 180.464 109.783) (end 180.464 106.84) (width 1) (layer "B.Cu") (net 4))
 (segment (start 170.603 119.644) (end 180.464 109.783) (width 1) (layer "B.Cu") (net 4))
 (segment (start 180.464 106.84) (end 180.448 106.824) (width 1) (layer "B.Cu") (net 4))
 (segment (start 194.18 104.83) (end 194.18 101.026) (width 1) (layer "B.Cu") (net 4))
 (segment (start 194.18 101.026) (end 194.178 101.024) (width 1) (layer "B.Cu") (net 4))
 (segment (start 177.924 129.668) (end 177.908 129.684) (width 1) (layer "B.Cu") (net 6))
 (segment (start 200.022 79.811) (end 198.371 79.811) (width 1) (layer "B.Cu") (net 6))
 (segment (start 177.924 126.928) (end 201.8 103.052) (width 1) (layer "B.Cu") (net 6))
 (segment (start 201.8 81.589) (end 200.022 79.811) (width 1) (layer "B.Cu") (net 6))
 (segment (start 177.924 126.928) (end 177.924 129.668) (width 1) (layer "B.Cu") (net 6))
 (segment (start 175.72 124.724) (end 177.924 126.928) (width 1) (layer "B.Cu") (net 6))
 (segment (start 201.8 103.052) (end 201.8 81.589) (width 1) (layer "B.Cu") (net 6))
 (segment (start 163.043 124.724) (end 175.72 124.724) (width 1) (layer "B.Cu") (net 6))
 (segment (start 198.371 79.811) (end 196.718 78.158) (width 1) (layer "B.Cu") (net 6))
 (segment (start 196.718 78.158) (end 196.718 75.624) (width 1) (layer "B.Cu") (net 6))
 (segment (start 168.78 78.287) (end 151.508 78.287) (width 1) (layer "F.Cu") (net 30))
 (segment (start 144.142 102.671) (end 145.92 104.449) (width 1) (layer "F.Cu") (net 30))
 (segment (start 151.508 78.287) (end 144.142 86.923) (width 1) (layer "F.Cu") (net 30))
 (segment (start 145.92 104.449) (end 172.844 104.449) (width 1) (layer "F.Cu") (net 30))
 (segment (start 144.142 86.923) (end 144.142 102.671) (width 1) (layer "F.Cu") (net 30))
 (via (at 172.844 104.449) (size 2) (drill 0.8) (layers "F.Cu" "B.Cu") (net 30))
 (via (at 168.78 78.287) (size 2) (drill 0.8) (layers "F.Cu" "B.Cu") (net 30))
 (segment (start 172.828 106.824) (end 172.828 104.465) (width 1) (layer "B.Cu") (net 30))
 (segment (start 168.78 75.626) (end 168.778 75.624) (width 1) (layer "B.Cu") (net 30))
 (segment (start 172.828 104.465) (end 172.844 104.449) (width 1) (layer "B.Cu") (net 30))
 (segment (start 168.78 78.287) (end 168.78 75.626) (width 1) (layer "B.Cu") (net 30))
 (segment (start 150.998 68.002) (end 151 68) (width 2) (layer "B.Cu") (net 36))
 (segment (start 150.998 75.624) (end 150.998 68.002) (width 2) (layer "B.Cu") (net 36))
 (segment (start 163.7 65.48) (end 151.02 65.48) (width 2) (layer "B.Cu") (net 42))
 (segment (start 151.02 65.48) (end 151 65.5) (width 2) (layer "B.Cu") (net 42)))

